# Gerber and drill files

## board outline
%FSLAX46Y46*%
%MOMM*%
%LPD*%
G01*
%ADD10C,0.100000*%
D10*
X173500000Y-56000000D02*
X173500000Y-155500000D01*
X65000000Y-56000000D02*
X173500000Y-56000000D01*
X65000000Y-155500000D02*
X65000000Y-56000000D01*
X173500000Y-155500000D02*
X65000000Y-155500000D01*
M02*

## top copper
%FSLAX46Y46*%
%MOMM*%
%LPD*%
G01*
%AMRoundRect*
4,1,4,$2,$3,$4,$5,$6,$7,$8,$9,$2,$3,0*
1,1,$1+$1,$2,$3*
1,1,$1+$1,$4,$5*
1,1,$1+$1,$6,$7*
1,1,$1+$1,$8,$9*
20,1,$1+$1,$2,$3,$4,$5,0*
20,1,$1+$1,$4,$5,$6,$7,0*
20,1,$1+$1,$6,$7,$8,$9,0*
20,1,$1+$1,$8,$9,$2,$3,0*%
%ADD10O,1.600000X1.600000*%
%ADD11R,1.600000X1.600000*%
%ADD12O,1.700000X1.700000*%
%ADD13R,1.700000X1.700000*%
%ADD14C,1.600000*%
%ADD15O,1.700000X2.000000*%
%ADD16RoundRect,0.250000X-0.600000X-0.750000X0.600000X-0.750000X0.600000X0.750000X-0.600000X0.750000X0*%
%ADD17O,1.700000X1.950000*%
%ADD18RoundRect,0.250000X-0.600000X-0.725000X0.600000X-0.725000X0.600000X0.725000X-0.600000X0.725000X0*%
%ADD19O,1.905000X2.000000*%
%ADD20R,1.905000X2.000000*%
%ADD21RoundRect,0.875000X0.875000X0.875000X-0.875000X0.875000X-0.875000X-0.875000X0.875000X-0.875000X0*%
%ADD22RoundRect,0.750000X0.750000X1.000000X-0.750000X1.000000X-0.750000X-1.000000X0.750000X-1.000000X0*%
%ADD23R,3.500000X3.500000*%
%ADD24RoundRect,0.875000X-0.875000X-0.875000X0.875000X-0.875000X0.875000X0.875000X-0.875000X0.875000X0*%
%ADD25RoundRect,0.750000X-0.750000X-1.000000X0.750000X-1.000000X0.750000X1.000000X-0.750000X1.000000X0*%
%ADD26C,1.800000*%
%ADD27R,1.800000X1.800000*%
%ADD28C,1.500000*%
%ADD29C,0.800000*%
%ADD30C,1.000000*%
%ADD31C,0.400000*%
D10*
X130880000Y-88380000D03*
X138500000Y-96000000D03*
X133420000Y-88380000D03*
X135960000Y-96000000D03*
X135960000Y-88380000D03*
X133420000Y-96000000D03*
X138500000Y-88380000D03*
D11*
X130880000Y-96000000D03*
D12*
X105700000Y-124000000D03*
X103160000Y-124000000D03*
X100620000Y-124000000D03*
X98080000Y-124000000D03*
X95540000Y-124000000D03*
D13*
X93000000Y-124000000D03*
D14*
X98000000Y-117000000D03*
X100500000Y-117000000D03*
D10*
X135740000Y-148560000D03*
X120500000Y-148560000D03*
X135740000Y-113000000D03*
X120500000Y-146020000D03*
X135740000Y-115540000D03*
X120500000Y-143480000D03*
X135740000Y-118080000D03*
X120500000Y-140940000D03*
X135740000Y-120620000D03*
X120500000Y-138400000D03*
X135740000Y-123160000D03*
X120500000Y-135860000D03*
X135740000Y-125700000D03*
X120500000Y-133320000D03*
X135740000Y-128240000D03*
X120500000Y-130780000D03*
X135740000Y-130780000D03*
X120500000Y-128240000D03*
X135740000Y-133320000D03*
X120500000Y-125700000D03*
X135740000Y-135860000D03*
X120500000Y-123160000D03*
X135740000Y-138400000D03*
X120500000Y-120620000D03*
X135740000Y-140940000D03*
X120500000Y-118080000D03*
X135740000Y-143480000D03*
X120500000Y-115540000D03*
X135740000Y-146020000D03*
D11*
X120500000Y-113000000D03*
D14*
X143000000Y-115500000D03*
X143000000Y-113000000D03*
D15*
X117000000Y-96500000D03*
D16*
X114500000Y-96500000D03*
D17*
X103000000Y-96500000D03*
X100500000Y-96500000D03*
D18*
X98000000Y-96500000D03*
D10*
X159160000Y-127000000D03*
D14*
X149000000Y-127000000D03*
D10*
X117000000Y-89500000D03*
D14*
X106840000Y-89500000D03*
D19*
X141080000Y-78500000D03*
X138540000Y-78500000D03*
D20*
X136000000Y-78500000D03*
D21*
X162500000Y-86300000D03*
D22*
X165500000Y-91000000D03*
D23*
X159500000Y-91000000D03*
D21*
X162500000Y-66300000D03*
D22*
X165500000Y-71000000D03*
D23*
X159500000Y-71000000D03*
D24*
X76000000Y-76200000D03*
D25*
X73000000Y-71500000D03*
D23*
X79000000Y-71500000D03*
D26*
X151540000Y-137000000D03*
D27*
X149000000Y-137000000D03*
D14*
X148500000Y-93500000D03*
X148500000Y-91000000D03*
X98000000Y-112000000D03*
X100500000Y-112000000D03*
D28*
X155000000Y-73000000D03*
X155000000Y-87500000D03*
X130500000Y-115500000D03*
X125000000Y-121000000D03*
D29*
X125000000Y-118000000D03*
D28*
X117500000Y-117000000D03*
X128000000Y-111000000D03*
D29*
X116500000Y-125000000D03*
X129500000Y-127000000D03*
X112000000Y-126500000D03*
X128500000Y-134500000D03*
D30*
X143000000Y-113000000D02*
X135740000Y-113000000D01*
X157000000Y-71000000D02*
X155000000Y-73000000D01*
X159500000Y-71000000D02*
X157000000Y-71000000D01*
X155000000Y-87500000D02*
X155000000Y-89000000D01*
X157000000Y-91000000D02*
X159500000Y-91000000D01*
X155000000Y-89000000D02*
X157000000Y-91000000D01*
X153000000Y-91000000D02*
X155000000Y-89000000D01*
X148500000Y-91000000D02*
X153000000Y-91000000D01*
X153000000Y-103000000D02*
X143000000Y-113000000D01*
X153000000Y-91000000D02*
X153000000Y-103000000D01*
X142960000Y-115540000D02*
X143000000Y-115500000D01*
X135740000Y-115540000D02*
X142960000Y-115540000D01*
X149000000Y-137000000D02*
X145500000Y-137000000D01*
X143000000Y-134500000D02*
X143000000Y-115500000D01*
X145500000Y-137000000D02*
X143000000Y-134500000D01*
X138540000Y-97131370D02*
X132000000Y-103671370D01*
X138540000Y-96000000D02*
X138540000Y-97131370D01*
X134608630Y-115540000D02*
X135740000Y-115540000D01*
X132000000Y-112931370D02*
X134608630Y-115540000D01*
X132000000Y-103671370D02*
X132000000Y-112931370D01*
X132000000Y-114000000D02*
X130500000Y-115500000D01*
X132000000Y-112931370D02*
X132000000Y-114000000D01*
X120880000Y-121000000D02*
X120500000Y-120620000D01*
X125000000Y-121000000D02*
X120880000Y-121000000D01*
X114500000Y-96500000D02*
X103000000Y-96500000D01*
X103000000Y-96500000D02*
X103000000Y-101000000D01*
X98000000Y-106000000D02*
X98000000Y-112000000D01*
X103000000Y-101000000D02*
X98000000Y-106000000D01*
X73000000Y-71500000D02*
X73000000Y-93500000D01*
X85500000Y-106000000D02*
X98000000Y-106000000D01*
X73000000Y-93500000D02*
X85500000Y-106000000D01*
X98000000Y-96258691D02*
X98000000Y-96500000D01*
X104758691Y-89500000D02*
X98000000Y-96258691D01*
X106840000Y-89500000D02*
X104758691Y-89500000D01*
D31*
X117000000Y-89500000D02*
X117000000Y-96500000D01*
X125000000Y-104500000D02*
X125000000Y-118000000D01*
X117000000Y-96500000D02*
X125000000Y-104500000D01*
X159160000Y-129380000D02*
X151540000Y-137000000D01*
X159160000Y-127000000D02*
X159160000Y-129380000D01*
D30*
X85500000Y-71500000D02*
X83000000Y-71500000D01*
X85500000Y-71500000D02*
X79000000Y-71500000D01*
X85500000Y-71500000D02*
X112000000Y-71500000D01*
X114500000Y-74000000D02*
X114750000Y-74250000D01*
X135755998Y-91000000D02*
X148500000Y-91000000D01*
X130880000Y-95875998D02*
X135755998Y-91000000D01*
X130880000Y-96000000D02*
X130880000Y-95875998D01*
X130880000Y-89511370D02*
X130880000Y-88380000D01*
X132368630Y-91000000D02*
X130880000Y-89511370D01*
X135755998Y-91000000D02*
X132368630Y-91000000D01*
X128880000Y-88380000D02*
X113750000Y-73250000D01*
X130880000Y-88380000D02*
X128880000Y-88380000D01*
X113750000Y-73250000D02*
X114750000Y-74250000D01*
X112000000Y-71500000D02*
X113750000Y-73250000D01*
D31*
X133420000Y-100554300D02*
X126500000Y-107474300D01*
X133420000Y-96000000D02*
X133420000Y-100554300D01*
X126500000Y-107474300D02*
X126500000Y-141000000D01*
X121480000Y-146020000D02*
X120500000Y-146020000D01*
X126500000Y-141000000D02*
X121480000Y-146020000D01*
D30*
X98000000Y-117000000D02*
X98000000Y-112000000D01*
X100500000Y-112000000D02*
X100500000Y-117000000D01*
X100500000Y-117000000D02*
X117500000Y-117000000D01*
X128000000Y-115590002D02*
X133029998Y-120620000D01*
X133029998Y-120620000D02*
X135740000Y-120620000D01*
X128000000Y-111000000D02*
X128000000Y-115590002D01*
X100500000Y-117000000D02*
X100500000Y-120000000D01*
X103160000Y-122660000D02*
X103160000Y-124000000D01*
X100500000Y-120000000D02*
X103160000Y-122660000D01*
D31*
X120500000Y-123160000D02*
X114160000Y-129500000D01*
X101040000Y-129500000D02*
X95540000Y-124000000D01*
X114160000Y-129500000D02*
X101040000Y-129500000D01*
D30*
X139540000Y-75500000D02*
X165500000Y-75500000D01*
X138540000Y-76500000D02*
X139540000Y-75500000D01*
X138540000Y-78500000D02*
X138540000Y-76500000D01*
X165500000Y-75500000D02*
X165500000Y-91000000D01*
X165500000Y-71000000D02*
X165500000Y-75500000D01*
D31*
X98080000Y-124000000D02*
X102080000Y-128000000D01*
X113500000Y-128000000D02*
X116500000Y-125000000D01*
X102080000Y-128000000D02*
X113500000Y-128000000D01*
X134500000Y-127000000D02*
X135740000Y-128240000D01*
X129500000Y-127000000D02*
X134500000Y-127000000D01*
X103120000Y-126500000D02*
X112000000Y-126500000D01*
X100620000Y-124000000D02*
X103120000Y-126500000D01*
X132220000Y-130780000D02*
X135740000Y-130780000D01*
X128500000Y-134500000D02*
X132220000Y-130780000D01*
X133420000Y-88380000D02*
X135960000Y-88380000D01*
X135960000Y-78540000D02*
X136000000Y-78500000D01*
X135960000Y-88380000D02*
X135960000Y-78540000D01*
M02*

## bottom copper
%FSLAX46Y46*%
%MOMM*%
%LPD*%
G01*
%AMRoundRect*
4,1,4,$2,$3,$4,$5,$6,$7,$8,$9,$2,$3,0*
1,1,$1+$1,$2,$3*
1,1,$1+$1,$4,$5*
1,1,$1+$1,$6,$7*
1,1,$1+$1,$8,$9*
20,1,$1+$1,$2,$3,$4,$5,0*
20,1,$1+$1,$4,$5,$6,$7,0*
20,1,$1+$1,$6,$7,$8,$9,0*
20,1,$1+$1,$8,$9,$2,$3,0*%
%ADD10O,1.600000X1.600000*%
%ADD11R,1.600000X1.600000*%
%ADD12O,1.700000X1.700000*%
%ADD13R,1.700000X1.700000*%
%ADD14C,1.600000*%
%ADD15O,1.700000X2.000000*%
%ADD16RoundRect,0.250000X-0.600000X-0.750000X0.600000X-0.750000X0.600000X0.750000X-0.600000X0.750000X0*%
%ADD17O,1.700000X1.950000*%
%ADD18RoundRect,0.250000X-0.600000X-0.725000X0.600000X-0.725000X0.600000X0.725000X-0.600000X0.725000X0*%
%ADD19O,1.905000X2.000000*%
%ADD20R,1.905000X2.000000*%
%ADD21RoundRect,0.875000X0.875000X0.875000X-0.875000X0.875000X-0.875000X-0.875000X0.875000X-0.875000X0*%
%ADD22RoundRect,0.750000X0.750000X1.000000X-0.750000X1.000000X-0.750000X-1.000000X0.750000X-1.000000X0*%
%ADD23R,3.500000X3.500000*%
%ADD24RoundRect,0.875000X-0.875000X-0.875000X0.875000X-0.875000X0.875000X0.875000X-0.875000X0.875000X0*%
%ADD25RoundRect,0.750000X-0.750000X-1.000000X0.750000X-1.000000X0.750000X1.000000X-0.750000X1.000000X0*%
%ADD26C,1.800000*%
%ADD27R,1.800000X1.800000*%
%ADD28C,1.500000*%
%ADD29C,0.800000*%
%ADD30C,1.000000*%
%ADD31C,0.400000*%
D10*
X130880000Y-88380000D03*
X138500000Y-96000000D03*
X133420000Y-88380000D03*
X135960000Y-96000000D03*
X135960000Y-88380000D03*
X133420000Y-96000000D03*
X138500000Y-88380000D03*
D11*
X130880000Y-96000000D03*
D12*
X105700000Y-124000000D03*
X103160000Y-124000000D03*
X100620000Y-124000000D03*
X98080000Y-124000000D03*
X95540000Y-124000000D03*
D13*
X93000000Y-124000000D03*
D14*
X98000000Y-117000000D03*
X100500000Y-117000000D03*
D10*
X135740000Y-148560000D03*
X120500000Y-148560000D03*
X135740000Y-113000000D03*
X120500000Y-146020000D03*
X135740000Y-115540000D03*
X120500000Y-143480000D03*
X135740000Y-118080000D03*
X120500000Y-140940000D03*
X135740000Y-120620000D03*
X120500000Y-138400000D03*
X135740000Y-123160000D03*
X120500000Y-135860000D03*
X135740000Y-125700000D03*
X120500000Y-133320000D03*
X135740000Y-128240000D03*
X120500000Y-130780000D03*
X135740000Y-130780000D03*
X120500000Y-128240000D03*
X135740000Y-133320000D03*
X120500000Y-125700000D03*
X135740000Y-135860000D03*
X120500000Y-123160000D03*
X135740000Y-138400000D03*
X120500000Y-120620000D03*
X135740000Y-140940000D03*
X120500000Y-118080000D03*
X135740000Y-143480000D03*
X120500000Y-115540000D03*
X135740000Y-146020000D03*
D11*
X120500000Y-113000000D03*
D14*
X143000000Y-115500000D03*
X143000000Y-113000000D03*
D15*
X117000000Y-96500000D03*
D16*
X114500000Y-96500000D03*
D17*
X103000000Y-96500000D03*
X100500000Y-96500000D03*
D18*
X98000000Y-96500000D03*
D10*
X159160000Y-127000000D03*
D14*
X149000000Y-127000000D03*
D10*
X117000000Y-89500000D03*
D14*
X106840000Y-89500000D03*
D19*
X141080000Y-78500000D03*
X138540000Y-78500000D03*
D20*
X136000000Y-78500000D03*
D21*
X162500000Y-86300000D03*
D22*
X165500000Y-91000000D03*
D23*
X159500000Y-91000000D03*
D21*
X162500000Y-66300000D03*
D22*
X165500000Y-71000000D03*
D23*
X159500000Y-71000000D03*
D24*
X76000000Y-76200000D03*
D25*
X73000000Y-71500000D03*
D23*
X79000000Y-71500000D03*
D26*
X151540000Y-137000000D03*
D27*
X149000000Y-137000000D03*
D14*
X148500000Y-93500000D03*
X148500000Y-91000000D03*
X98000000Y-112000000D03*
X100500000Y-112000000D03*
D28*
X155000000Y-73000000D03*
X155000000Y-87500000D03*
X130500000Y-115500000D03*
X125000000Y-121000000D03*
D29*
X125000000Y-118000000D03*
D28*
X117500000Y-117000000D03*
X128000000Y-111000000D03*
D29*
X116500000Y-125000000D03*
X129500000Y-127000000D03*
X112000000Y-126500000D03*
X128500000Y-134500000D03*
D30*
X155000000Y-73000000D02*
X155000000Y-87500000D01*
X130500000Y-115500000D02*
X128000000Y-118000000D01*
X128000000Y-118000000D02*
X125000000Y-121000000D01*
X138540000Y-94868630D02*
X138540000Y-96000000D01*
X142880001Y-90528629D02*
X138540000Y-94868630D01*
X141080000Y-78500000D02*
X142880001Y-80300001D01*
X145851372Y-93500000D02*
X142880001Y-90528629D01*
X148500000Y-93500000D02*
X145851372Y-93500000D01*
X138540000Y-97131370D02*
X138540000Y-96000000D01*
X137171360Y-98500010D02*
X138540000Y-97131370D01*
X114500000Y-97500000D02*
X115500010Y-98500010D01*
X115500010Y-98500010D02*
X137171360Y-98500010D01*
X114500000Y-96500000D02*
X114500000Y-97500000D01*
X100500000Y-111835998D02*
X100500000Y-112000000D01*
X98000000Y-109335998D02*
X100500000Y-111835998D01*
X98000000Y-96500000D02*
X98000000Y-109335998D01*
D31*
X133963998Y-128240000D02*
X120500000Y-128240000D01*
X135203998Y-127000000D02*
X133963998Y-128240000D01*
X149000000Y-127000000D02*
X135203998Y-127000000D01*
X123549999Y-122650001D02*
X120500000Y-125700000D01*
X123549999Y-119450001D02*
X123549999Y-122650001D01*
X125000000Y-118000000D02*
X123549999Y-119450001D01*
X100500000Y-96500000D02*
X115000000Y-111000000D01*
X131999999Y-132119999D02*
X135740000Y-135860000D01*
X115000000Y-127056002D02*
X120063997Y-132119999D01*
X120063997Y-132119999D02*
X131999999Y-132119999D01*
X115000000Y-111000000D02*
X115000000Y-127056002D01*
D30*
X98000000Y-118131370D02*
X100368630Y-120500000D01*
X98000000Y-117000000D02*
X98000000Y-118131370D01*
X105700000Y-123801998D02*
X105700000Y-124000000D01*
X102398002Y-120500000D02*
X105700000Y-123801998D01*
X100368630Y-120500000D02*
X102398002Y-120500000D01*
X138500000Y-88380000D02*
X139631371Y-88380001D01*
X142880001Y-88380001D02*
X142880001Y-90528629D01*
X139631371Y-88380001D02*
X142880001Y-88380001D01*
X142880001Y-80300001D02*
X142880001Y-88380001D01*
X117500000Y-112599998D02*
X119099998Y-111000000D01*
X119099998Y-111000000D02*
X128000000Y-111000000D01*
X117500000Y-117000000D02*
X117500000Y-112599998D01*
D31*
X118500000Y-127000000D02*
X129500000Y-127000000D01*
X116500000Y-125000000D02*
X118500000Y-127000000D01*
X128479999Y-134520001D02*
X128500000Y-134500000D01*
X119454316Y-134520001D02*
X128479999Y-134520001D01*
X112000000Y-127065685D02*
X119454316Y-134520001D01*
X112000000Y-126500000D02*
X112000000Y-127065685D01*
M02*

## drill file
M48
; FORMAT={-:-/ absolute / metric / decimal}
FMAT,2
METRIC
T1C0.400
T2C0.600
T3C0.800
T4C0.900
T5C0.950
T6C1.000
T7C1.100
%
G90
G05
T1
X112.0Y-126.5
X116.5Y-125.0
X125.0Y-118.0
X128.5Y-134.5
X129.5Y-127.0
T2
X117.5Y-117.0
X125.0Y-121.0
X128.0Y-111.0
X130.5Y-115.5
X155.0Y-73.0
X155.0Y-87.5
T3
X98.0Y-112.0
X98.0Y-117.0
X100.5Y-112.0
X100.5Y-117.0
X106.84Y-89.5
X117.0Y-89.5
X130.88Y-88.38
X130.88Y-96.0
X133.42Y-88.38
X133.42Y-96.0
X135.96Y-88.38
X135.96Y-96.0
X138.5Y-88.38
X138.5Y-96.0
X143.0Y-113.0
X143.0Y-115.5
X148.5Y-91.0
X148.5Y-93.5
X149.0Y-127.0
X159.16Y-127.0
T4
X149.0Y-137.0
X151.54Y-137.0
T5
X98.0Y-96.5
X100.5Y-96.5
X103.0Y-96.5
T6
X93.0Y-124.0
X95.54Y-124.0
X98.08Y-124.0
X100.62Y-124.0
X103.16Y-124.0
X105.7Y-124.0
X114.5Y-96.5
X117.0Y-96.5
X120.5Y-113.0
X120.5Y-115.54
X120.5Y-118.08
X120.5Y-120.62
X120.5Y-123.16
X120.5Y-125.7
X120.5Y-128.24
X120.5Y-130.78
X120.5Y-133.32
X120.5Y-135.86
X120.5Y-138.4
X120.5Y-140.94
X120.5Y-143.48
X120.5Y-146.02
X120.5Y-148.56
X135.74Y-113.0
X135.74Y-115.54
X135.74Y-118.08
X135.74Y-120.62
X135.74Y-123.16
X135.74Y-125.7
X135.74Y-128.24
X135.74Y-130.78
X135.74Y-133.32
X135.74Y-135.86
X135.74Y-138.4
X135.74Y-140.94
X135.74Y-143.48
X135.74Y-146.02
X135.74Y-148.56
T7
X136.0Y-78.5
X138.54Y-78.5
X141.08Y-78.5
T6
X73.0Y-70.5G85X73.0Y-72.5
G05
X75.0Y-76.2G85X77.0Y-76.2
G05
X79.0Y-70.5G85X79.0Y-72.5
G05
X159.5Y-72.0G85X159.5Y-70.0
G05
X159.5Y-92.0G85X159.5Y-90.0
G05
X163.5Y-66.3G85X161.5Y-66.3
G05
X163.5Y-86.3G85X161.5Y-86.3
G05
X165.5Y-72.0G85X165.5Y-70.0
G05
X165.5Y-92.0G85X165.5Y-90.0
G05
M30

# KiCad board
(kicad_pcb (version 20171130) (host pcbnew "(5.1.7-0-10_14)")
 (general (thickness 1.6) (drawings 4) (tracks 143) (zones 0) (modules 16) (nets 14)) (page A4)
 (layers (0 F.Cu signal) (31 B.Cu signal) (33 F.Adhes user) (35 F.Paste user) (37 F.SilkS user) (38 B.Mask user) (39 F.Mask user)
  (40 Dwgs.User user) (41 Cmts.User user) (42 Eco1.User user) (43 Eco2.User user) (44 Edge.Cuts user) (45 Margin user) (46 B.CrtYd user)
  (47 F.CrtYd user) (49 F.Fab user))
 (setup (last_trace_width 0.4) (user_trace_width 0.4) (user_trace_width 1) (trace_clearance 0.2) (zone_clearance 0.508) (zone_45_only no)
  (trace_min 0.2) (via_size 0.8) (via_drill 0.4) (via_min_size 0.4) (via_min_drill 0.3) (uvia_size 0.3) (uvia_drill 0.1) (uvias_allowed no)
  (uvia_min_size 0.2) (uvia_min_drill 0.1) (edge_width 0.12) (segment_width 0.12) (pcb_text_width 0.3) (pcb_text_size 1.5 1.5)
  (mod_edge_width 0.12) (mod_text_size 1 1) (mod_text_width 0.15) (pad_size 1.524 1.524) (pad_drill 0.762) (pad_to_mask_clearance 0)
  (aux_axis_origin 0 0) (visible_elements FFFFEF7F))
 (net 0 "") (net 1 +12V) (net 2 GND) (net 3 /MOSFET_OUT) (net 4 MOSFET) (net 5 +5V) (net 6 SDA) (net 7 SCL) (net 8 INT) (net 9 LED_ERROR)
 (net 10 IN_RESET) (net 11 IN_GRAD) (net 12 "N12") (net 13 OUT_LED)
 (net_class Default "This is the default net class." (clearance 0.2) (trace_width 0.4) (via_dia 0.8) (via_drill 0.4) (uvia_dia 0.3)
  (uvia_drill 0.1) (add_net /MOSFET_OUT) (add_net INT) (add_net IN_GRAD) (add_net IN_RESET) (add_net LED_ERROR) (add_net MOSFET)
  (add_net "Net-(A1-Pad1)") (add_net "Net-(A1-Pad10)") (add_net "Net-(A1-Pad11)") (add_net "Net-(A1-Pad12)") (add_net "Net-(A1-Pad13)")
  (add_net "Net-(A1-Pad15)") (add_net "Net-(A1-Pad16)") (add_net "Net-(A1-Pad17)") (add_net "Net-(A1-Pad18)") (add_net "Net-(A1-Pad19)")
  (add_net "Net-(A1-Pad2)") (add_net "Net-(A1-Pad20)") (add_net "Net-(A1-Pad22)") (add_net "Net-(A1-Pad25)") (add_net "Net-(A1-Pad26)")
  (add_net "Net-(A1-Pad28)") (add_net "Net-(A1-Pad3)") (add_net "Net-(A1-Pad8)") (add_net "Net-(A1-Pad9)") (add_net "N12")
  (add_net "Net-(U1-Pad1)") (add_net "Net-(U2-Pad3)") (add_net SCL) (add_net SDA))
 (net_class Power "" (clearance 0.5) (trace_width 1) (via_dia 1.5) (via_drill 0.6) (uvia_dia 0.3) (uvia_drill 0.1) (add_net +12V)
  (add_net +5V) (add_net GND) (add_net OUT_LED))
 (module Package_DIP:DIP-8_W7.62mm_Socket (layer F.Cu) (at 130.88 96 90)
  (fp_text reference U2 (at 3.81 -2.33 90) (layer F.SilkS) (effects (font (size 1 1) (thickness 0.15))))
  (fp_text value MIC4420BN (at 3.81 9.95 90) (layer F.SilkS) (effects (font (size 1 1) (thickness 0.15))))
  (pad 8 thru_hole oval (at 7.62 0 90) (size 1.6 1.6) (drill 0.8) (layers *.Cu *.Mask) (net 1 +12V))
  (pad 4 thru_hole oval (at 0 7.62 90) (size 1.6 1.6) (drill 0.8) (layers *.Cu *.Mask) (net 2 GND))
  (pad 7 thru_hole oval (at 7.62 2.54 90) (size 1.6 1.6) (drill 0.8) (layers *.Cu *.Mask) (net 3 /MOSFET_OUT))
  (pad 3 thru_hole oval (at 0 5.08 90) (size 1.6 1.6) (drill 0.8) (layers *.Cu *.Mask))
  (pad 6 thru_hole oval (at 7.62 5.08 90) (size 1.6 1.6) (drill 0.8) (layers *.Cu *.Mask) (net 3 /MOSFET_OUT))
  (pad 2 thru_hole oval (at 0 2.54 90) (size 1.6 1.6) (drill 0.8) (layers *.Cu *.Mask) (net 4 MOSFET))
  (pad 5 thru_hole oval (at 7.62 7.62 90) (size 1.6 1.6) (drill 0.8) (layers *.Cu *.Mask) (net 2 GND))
  (pad 1 thru_hole rect (at 0 0 90) (size 1.6 1.6) (drill 0.8) (layers *.Cu *.Mask) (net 1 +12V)))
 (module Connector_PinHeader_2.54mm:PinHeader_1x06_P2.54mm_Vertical (layer F.Cu) (at 93 124 90)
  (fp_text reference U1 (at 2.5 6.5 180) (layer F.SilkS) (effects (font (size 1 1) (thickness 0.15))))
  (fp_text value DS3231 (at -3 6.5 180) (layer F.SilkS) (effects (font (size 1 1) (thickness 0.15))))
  (pad 6 thru_hole oval (at 0 12.7 90) (size 1.7 1.7) (drill 1) (layers *.Cu *.Mask) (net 2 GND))
  (pad 5 thru_hole oval (at 0 10.16 90) (size 1.7 1.7) (drill 1) (layers *.Cu *.Mask) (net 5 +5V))
  (pad 4 thru_hole oval (at 0 7.62 90) (size 1.7 1.7) (drill 1) (layers *.Cu *.Mask) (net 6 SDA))
  (pad 3 thru_hole oval (at 0 5.08 90) (size 1.7 1.7) (drill 1) (layers *.Cu *.Mask) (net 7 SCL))
  (pad 2 thru_hole oval (at 0 2.54 90) (size 1.7 1.7) (drill 1) (layers *.Cu *.Mask) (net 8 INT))
  (pad 1 thru_hole rect (at 0 0 90) (size 1.7 1.7) (drill 1) (layers *.Cu *.Mask)))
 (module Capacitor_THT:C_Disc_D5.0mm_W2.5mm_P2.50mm (layer F.Cu) (at 100.5 117 180)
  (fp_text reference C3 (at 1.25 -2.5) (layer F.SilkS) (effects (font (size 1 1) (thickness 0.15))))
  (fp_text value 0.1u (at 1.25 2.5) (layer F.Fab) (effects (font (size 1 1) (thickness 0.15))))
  (pad 2 thru_hole circle (at 2.5 0 180) (size 1.6 1.6) (drill 0.8) (layers *.Cu *.Mask) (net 2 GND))
  (pad 1 thru_hole circle (at 0 0 180) (size 1.6 1.6) (drill 0.8) (layers *.Cu *.Mask) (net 5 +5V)))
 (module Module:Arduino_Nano (layer F.Cu) (at 120.5 113)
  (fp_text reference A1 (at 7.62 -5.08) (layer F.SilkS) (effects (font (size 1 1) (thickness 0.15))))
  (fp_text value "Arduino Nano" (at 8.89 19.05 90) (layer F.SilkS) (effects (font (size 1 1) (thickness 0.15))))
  (pad 16 thru_hole oval (at 15.24 35.56) (size 1.6 1.6) (drill 1) (layers *.Cu *.Mask))
  (pad 15 thru_hole oval (at 0 35.56) (size 1.6 1.6) (drill 1) (layers *.Cu *.Mask))
  (pad 30 thru_hole oval (at 15.24 0) (size 1.6 1.6) (drill 1) (layers *.Cu *.Mask) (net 1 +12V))
  (pad 14 thru_hole oval (at 0 33.02) (size 1.6 1.6) (drill 1) (layers *.Cu *.Mask) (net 4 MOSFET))
  (pad 29 thru_hole oval (at 15.24 2.54) (size 1.6 1.6) (drill 1) (layers *.Cu *.Mask) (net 2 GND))
  (pad 13 thru_hole oval (at 0 30.48) (size 1.6 1.6) (drill 1) (layers *.Cu *.Mask))
  (pad 28 thru_hole oval (at 15.24 5.08) (size 1.6 1.6) (drill 1) (layers *.Cu *.Mask))
  (pad 12 thru_hole oval (at 0 27.94) (size 1.6 1.6) (drill 1) (layers *.Cu *.Mask))
  (pad 27 thru_hole oval (at 15.24 7.62) (size 1.6 1.6) (drill 1) (layers *.Cu *.Mask) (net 5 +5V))
  (pad 11 thru_hole oval (at 0 25.4) (size 1.6 1.6) (drill 1) (layers *.Cu *.Mask))
  (pad 26 thru_hole oval (at 15.24 10.16) (size 1.6 1.6) (drill 1) (layers *.Cu *.Mask))
  (pad 10 thru_hole oval (at 0 22.86) (size 1.6 1.6) (drill 1) (layers *.Cu *.Mask))
  (pad 25 thru_hole oval (at 15.24 12.7) (size 1.6 1.6) (drill 1) (layers *.Cu *.Mask))
  (pad 9 thru_hole oval (at 0 20.32) (size 1.6 1.6) (drill 1) (layers *.Cu *.Mask))
  (pad 24 thru_hole oval (at 15.24 15.24) (size 1.6 1.6) (drill 1) (layers *.Cu *.Mask) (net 7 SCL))
  (pad 8 thru_hole oval (at 0 17.78) (size 1.6 1.6) (drill 1) (layers *.Cu *.Mask))
  (pad 23 thru_hole oval (at 15.24 17.78) (size 1.6 1.6) (drill 1) (layers *.Cu *.Mask) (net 6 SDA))
  (pad 7 thru_hole oval (at 0 15.24) (size 1.6 1.6) (drill 1) (layers *.Cu *.Mask) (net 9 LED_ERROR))
  (pad 22 thru_hole oval (at 15.24 20.32) (size 1.6 1.6) (drill 1) (layers *.Cu *.Mask))
  (pad 6 thru_hole oval (at 0 12.7) (size 1.6 1.6) (drill 1) (layers *.Cu *.Mask) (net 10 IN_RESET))
  (pad 21 thru_hole oval (at 15.24 22.86) (size 1.6 1.6) (drill 1) (layers *.Cu *.Mask) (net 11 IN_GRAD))
  (pad 5 thru_hole oval (at 0 10.16) (size 1.6 1.6) (drill 1) (layers *.Cu *.Mask) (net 8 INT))
  (pad 20 thru_hole oval (at 15.24 25.4) (size 1.6 1.6) (drill 1) (layers *.Cu *.Mask))
  (pad 4 thru_hole oval (at 0 7.62) (size 1.6 1.6) (drill 1) (layers *.Cu *.Mask) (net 2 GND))
  (pad 19 thru_hole oval (at 15.24 27.94) (size 1.6 1.6) (drill 1) (layers *.Cu *.Mask))
  (pad 3 thru_hole oval (at 0 5.08) (size 1.6 1.6) (drill 1) (layers *.Cu *.Mask))
  (pad 18 thru_hole oval (at 15.24 30.48) (size 1.6 1.6) (drill 1) (layers *.Cu *.Mask))
  (pad 2 thru_hole oval (at 0 2.54) (size 1.6 1.6) (drill 1) (layers *.Cu *.Mask))
  (pad 17 thru_hole oval (at 15.24 33.02) (size 1.6 1.6) (drill 1) (layers *.Cu *.Mask))
  (pad 1 thru_hole rect (at 0 0) (size 1.6 1.6) (drill 1) (layers *.Cu *.Mask)))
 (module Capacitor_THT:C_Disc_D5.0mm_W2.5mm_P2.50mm (layer F.Cu) (at 143 113 270)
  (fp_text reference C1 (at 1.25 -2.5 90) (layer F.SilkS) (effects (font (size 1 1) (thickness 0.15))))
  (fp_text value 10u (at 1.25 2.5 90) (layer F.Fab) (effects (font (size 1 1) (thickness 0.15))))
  (pad 2 thru_hole circle (at 2.5 0 270) (size 1.6 1.6) (drill 0.8) (layers *.Cu *.Mask) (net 2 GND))
  (pad 1 thru_hole circle (at 0 0 270) (size 1.6 1.6) (drill 0.8) (layers *.Cu *.Mask) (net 1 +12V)))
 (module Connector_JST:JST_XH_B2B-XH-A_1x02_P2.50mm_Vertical (layer F.Cu) (at 114.5 96.5)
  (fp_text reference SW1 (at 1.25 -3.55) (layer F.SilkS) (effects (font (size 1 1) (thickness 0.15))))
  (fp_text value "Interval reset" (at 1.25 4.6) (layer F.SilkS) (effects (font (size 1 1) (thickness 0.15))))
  (pad 2 thru_hole oval (at 2.5 0) (size 1.7 2) (drill 1) (layers *.Cu *.Mask) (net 10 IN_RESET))
  (pad 1 thru_hole roundrect (at 0 0) (size 1.7 2) (drill 1) (layers *.Cu *.Mask) (roundrect_rratio 0.147059) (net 2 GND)))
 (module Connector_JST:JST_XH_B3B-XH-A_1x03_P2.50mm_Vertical (layer F.Cu) (at 98 96.5)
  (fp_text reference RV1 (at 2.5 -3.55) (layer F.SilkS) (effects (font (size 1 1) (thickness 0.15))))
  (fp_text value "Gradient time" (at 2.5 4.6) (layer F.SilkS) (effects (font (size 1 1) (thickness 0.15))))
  (pad 3 thru_hole oval (at 5 0) (size 1.7 1.95) (drill 0.95) (layers *.Cu *.Mask) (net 2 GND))
  (pad 2 thru_hole oval (at 2.5 0) (size 1.7 1.95) (drill 0.95) (layers *.Cu *.Mask) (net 11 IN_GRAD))
  (pad 1 thru_hole roundrect (at 0 0) (size 1.7 1.95) (drill 0.95) (layers *.Cu *.Mask) (roundrect_rratio 0.147059) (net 5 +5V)))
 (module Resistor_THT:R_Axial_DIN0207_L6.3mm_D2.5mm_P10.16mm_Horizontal (layer F.Cu) (at 149 127)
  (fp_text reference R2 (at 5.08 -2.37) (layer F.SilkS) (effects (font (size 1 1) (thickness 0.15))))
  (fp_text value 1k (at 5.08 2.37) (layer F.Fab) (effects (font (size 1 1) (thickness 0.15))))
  (pad 2 thru_hole oval (at 10.16 0) (size 1.6 1.6) (drill 0.8) (layers *.Cu *.Mask) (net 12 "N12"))
  (pad 1 thru_hole circle (at 0 0) (size 1.6 1.6) (drill 0.8) (layers *.Cu *.Mask) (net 9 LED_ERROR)))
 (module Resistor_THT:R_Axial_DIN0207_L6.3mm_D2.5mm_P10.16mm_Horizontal (layer F.Cu) (at 106.84 89.5)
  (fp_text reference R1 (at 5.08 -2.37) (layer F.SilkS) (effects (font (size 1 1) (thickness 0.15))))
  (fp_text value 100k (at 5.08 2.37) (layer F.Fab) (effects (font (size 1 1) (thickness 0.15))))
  (pad 2 thru_hole oval (at 10.16 0) (size 1.6 1.6) (drill 0.8) (layers *.Cu *.Mask) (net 10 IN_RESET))
  (pad 1 thru_hole circle (at 0 0) (size 1.6 1.6) (drill 0.8) (layers *.Cu *.Mask) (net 5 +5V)))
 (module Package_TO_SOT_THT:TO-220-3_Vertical (layer F.Cu) (at 136 78.5)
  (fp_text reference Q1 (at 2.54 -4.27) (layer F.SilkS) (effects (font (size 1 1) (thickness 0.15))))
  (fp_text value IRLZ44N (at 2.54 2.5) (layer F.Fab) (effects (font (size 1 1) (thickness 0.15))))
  (pad 3 thru_hole oval (at 5.08 0) (size 1.905 2) (drill 1.1) (layers *.Cu *.Mask) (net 2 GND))
  (pad 2 thru_hole oval (at 2.54 0) (size 1.905 2) (drill 1.1) (layers *.Cu *.Mask) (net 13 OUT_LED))
  (pad 1 thru_hole rect (at 0 0) (size 1.905 2) (drill 1.1) (layers *.Cu *.Mask) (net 3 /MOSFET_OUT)))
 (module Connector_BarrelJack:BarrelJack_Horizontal (layer F.Cu) (at 159.5 91 180)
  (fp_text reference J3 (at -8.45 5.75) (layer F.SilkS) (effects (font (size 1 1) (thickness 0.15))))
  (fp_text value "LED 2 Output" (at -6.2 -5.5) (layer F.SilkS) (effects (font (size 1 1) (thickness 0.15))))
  (pad 3 thru_hole roundrect (at -3 4.7 180) (size 3.5 3.5) (drill oval 3 1) (layers *.Cu *.Mask) (roundrect_rratio 0.25))
  (pad 2 thru_hole roundrect (at -6 0 180) (size 3 3.5) (drill oval 1 3) (layers *.Cu *.Mask) (roundrect_rratio 0.25) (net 13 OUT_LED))
  (pad 1 thru_hole rect (at 0 0 180) (size 3.5 3.5) (drill oval 1 3) (layers *.Cu *.Mask) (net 1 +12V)))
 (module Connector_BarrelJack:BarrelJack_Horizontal (layer F.Cu) (at 159.5 71 180)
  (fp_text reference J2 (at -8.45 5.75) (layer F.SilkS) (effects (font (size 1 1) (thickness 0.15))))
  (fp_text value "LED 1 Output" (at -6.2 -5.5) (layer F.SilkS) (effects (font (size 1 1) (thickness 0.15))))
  (pad 3 thru_hole roundrect (at -3 4.7 180) (size 3.5 3.5) (drill oval 3 1) (layers *.Cu *.Mask) (roundrect_rratio 0.25))
  (pad 2 thru_hole roundrect (at -6 0 180) (size 3 3.5) (drill oval 1 3) (layers *.Cu *.Mask) (roundrect_rratio 0.25) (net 13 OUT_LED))
  (pad 1 thru_hole rect (at 0 0 180) (size 3.5 3.5) (drill oval 1 3) (layers *.Cu *.Mask) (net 1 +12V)))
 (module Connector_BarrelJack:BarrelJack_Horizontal (layer F.Cu) (at 79 71.5)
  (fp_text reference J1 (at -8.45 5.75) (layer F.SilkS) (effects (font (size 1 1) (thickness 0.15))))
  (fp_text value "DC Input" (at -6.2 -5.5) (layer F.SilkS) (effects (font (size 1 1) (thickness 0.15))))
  (pad 3 thru_hole roundrect (at -3 4.7) (size 3.5 3.5) (drill oval 3 1) (layers *.Cu *.Mask) (roundrect_rratio 0.25))
  (pad 2 thru_hole roundrect (at -6 0) (size 3 3.5) (drill oval 1 3) (layers *.Cu *.Mask) (roundrect_rratio 0.25) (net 2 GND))
  (pad 1 thru_hole rect (at 0 0) (size 3.5 3.5) (drill oval 1 3) (layers *.Cu *.Mask) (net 1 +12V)))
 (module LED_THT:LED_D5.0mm (layer F.Cu) (at 149 137)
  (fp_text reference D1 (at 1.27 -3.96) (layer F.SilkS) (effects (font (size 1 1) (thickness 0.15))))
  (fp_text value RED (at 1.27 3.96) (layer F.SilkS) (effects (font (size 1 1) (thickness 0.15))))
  (pad 2 thru_hole circle (at 2.54 0) (size 1.8 1.8) (drill 0.9) (layers *.Cu *.Mask) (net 12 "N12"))
  (pad 1 thru_hole rect (at 0 0) (size 1.8 1.8) (drill 0.9) (layers *.Cu *.Mask) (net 2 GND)))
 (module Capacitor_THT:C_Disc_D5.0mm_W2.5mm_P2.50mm (layer F.Cu) (at 148.5 91 270)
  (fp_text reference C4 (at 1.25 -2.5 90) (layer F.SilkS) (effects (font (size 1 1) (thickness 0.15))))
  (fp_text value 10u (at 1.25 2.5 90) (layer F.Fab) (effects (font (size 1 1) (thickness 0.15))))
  (pad 2 thru_hole circle (at 2.5 0 270) (size 1.6 1.6) (drill 0.8) (layers *.Cu *.Mask) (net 2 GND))
  (pad 1 thru_hole circle (at 0 0 270) (size 1.6 1.6) (drill 0.8) (layers *.Cu *.Mask) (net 1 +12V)))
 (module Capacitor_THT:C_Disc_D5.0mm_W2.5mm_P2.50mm (layer F.Cu) (at 100.5 112 180)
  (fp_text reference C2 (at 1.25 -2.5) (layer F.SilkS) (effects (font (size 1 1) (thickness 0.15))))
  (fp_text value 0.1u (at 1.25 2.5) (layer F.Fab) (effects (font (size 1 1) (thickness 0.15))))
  (pad 2 thru_hole circle (at 2.5 0 180) (size 1.6 1.6) (drill 0.8) (layers *.Cu *.Mask) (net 2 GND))
  (pad 1 thru_hole circle (at 0 0 180) (size 1.6 1.6) (drill 0.8) (layers *.Cu *.Mask) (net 5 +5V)))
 (gr_line (start 173.5 56) (end 173.5 155.5) (layer Edge.Cuts) (width 0.1))
 (gr_line (start 65 56) (end 173.5 56) (layer Edge.Cuts) (width 0.1))
 (gr_line (start 65 155.5) (end 65 56) (layer Edge.Cuts) (width 0.1))
 (gr_line (start 173.5 155.5) (end 65 155.5) (layer Edge.Cuts) (width 0.1))
 (segment (start 143 113) (end 135.74 113) (width 1) (layer F.Cu) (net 1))
 (via (at 155 73) (size 1.5) (drill 0.6) (layers F.Cu B.Cu) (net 1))
 (segment (start 157 71) (end 155 73) (width 1) (layer F.Cu) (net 1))
 (segment (start 159.5 71) (end 157 71) (width 1) (layer F.Cu) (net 1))
 (via (at 155 87.5) (size 1.5) (drill 0.6) (layers F.Cu B.Cu) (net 1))
 (segment (start 155 73) (end 155 87.5) (width 1) (layer B.Cu) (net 1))
 (segment (start 155 87.5) (end 155 89) (width 1) (layer F.Cu) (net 1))
 (segment (start 157 91) (end 159.5 91) (width 1) (layer F.Cu) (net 1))
 (segment (start 155 89) (end 157 91) (width 1) (layer F.Cu) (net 1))
 (segment (start 153 91) (end 155 89) (width 1) (layer F.Cu) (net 1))
 (segment (start 148.5 91) (end 153 91) (width 1) (layer F.Cu) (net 1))
 (segment (start 153 103) (end 143 113) (width 1) (layer F.Cu) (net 1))
 (segment (start 153 91) (end 153 103) (width 1) (layer F.Cu) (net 1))
 (segment (start 142.96 115.54) (end 143 115.5) (width 1) (layer F.Cu) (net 2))
 (segment (start 135.74 115.54) (end 142.96 115.54) (width 1) (layer F.Cu) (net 2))
 (segment (start 149 137) (end 145.5 137) (width 1) (layer F.Cu) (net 2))
 (segment (start 143 134.5) (end 143 115.5) (width 1) (layer F.Cu) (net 2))
 (segment (start 145.5 137) (end 143 134.5) (width 1) (layer F.Cu) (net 2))
 (segment (start 138.54 97.13137) (end 132 103.67137) (width 1) (layer F.Cu) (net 2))
 (segment (start 138.54 96) (end 138.54 97.13137) (width 1) (layer F.Cu) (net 2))
 (segment (start 134.60863 115.54) (end 135.74 115.54) (width 1) (layer F.Cu) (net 2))
 (segment (start 132 112.93137) (end 134.60863 115.54) (width 1) (layer F.Cu) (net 2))
 (segment (start 132 103.67137) (end 132 112.93137) (width 1) (layer F.Cu) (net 2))
 (via (at 130.5 115.5) (size 1.5) (drill 0.6) (layers F.Cu B.Cu) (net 2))
 (segment (start 132 114) (end 130.5 115.5) (width 1) (layer F.Cu) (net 2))
 (segment (start 132 112.93137) (end 132 114) (width 1) (layer F.Cu) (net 2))
 (segment (start 130.5 115.5) (end 128 118) (width 1) (layer B.Cu) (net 2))
 (via (at 125 121) (size 1.5) (drill 0.6) (layers F.Cu B.Cu) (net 2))
 (segment (start 128 118) (end 125 121) (width 1) (layer B.Cu) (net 2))
 (segment (start 120.88 121) (end 120.5 120.62) (width 1) (layer F.Cu) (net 2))
 (segment (start 125 121) (end 120.88 121) (width 1) (layer F.Cu) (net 2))
 (segment (start 114.5 96.5) (end 103 96.5) (width 1) (layer F.Cu) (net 2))
 (segment (start 103 96.5) (end 103 101) (width 1) (layer F.Cu) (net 2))
 (segment (start 98 106) (end 98 112) (width 1) (layer F.Cu) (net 2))
 (segment (start 103 101) (end 98 106) (width 1) (layer F.Cu) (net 2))
 (segment (start 73 71.5) (end 73 93.5) (width 1) (layer F.Cu) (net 2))
 (segment (start 85.5 106) (end 98 106) (width 1) (layer F.Cu) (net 2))
 (segment (start 73 93.5) (end 85.5 106) (width 1) (layer F.Cu) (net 2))
 (segment (start 138.54 94.86863) (end 138.54 96) (width 1) (layer B.Cu) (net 2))
 (segment (start 142.880001 90.528629) (end 138.54 94.86863) (width 1) (layer B.Cu) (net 2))
 (segment (start 141.08 78.5) (end 142.880001 80.300001) (width 1) (layer B.Cu) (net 2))
 (segment (start 145.851372 93.5) (end 142.880001 90.528629) (width 1) (layer B.Cu) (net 2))
 (segment (start 148.5 93.5) (end 145.851372 93.5) (width 1) (layer B.Cu) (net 2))
 (segment (start 138.54 97.13137) (end 138.54 96) (width 1) (layer B.Cu) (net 2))
 (segment (start 137.17136 98.50001) (end 138.54 97.13137) (width 1) (layer B.Cu) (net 2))
 (segment (start 114.5 97.5) (end 115.50001 98.50001) (width 1) (layer B.Cu) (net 2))
 (segment (start 115.50001 98.50001) (end 137.17136 98.50001) (width 1) (layer B.Cu) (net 2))
 (segment (start 114.5 96.5) (end 114.5 97.5) (width 1) (layer B.Cu) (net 2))
 (segment (start 98 96.258691) (end 98 96.5) (width 1) (layer F.Cu) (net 5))
 (segment (start 104.758691 89.5) (end 98 96.258691) (width 1) (layer F.Cu) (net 5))
 (segment (start 106.84 89.5) (end 104.758691 89.5) (width 1) (layer F.Cu) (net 5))
 (segment (start 100.5 111.835998) (end 100.5 112) (width 1) (layer B.Cu) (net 5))
 (segment (start 98 109.335998) (end 100.5 111.835998) (width 1) (layer B.Cu) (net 5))
 (segment (start 98 96.5) (end 98 109.335998) (width 1) (layer B.Cu) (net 5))
 (segment (start 133.963998 128.24) (end 120.5 128.24) (width 0.4) (layer B.Cu) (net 9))
 (segment (start 135.203998 127) (end 133.963998 128.24) (width 0.4) (layer B.Cu) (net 9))
 (segment (start 149 127) (end 135.203998 127) (width 0.4) (layer B.Cu) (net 9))
 (segment (start 117 89.5) (end 117 96.5) (width 0.4) (layer F.Cu) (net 10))
 (via (at 125 118) (size 0.8) (drill 0.4) (layers F.Cu B.Cu) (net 10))
 (segment (start 125 104.5) (end 125 118) (width 0.4) (layer F.Cu) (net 10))
 (segment (start 117 96.5) (end 125 104.5) (width 0.4) (layer F.Cu) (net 10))
 (segment (start 123.549999 122.650001) (end 120.5 125.7) (width 0.4) (layer B.Cu) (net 10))
 (segment (start 123.549999 119.450001) (end 123.549999 122.650001) (width 0.4) (layer B.Cu) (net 10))
 (segment (start 125 118) (end 123.549999 119.450001) (width 0.4) (layer B.Cu) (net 10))
 (segment (start 100.5 96.5) (end 115 111) (width 0.4) (layer B.Cu) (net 11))
 (segment (start 131.999999 132.119999) (end 135.74 135.86) (width 0.4) (layer B.Cu) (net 11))
 (segment (start 115 127.056002) (end 120.063997 132.119999) (width 0.4) (layer B.Cu) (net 11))
 (segment (start 120.063997 132.119999) (end 131.999999 132.119999) (width 0.4) (layer B.Cu) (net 11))
 (segment (start 115 111) (end 115 127.056002) (width 0.4) (layer B.Cu) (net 11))
 (segment (start 159.16 129.38) (end 151.54 137) (width 0.4) (layer F.Cu) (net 12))
 (segment (start 159.16 127) (end 159.16 129.38) (width 0.4) (layer F.Cu) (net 12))
 (segment (start 85.5 71.5) (end 83 71.5) (width 1) (layer F.Cu) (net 1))
 (segment (start 85.5 71.5) (end 79 71.5) (width 1) (layer F.Cu) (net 1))
 (segment (start 85.5 71.5) (end 112 71.5) (width 1) (layer F.Cu) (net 1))
 (segment (start 114.5 74) (end 114.75 74.25) (width 1) (layer F.Cu) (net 1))
 (segment (start 135.755998 91) (end 148.5 91) (width 1) (layer F.Cu) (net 1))
 (segment (start 130.88 95.875998) (end 135.755998 91) (width 1) (layer F.Cu) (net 1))
 (segment (start 130.88 96) (end 130.88 95.875998) (width 1) (layer F.Cu) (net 1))
 (segment (start 130.88 89.51137) (end 130.88 88.38) (width 1) (layer F.Cu) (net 1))
 (segment (start 132.36863 91) (end 130.88 89.51137) (width 1) (layer F.Cu) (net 1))
 (segment (start 135.755998 91) (end 132.36863 91) (width 1) (layer F.Cu) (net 1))
 (segment (start 128.88 88.38) (end 113.75 73.25) (width 1) (layer F.Cu) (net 1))
 (segment (start 130.88 88.38) (end 128.88 88.38) (width 1) (layer F.Cu) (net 1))
 (segment (start 113.75 73.25) (end 114.75 74.25) (width 1) (layer F.Cu) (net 1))
 (segment (start 112 71.5) (end 113.75 73.25) (width 1) (layer F.Cu) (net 1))
 (segment (start 133.42 100.5543) (end 126.5 107.4743) (width 0.4) (layer F.Cu) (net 4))
 (segment (start 133.42 96) (end 133.42 100.5543) (width 0.4) (layer F.Cu) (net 4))
 (segment (start 126.5 107.4743) (end 126.5 141) (width 0.4) (layer F.Cu) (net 4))
 (segment (start 121.48 146.02) (end 120.5 146.02) (width 0.4) (layer F.Cu) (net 4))
 (segment (start 126.5 141) (end 121.48 146.02) (width 0.4) (layer F.Cu) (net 4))
 (segment (start 98 117) (end 98 112) (width 1) (layer F.Cu) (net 2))
 (segment (start 98 118.13137) (end 100.36863 120.5) (width 1) (layer B.Cu) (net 2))
 (segment (start 98 117) (end 98 118.13137) (width 1) (layer B.Cu) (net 2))
 (segment (start 105.7 123.801998) (end 105.7 124) (width 1) (layer B.Cu) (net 2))
 (segment (start 102.398002 120.5) (end 105.7 123.801998) (width 1) (layer B.Cu) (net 2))
 (segment (start 100.36863 120.5) (end 102.398002 120.5) (width 1) (layer B.Cu) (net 2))
 (segment (start 138.5 88.38) (end 139.631371 88.380001) (width 1) (layer B.Cu) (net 2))
 (segment (start 142.880001 88.380001) (end 142.880001 90.528629) (width 1) (layer B.Cu) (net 2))
 (segment (start 139.631371 88.380001) (end 142.880001 88.380001) (width 1) (layer B.Cu) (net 2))
 (segment (start 142.880001 80.300001) (end 142.880001 88.380001) (width 1) (layer B.Cu) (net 2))
 (segment (start 100.5 112) (end 100.5 117) (width 1) (layer F.Cu) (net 5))
 (via (at 117.5 117) (size 1.5) (drill 0.6) (layers F.Cu B.Cu) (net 5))
 (segment (start 100.5 117) (end 117.5 117) (width 1) (layer F.Cu) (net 5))
 (segment (start 117.5 112.599998) (end 119.099998 111) (width 1) (layer B.Cu) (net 5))
 (via (at 128 111) (size 1.5) (drill 0.6) (layers F.Cu B.Cu) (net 5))
 (segment (start 119.099998 111) (end 128 111) (width 1) (layer B.Cu) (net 5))
 (segment (start 117.5 117) (end 117.5 112.599998) (width 1) (layer B.Cu) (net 5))
 (segment (start 128 115.590002) (end 133.029998 120.62) (width 1) (layer F.Cu) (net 5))
 (segment (start 133.029998 120.62) (end 135.74 120.62) (width 1) (layer F.Cu) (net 5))
 (segment (start 128 111) (end 128 115.590002) (width 1) (layer F.Cu) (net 5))
 (segment (start 100.5 117) (end 100.5 120) (width 1) (layer F.Cu) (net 5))
 (segment (start 103.16 122.66) (end 103.16 124) (width 1) (layer F.Cu) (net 5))
 (segment (start 100.5 120) (end 103.16 122.66) (width 1) (layer F.Cu) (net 5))
 (segment (start 120.5 123.16) (end 114.16 129.5) (width 0.4) (layer F.Cu) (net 8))
 (segment (start 101.04 129.5) (end 95.54 124) (width 0.4) (layer F.Cu) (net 8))
 (segment (start 114.16 129.5) (end 101.04 129.5) (width 0.4) (layer F.Cu) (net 8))
 (segment (start 139.54 75.5) (end 165.5 75.5) (width 1) (layer F.Cu) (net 13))
 (segment (start 138.54 76.5) (end 139.54 75.5) (width 1) (layer F.Cu) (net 13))
 (segment (start 138.54 78.5) (end 138.54 76.5) (width 1) (layer F.Cu) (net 13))
 (segment (start 165.5 75.5) (end 165.5 91) (width 1) (layer F.Cu) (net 13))
 (segment (start 165.5 71) (end 165.5 75.5) (width 1) (layer F.Cu) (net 13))
 (segment (start 98.08 124) (end 102.08 128) (width 0.4) (layer F.Cu) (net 7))
 (via (at 116.5 125) (size 0.8) (drill 0.4) (layers F.Cu B.Cu) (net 7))
 (segment (start 113.5 128) (end 116.5 125) (width 0.4) (layer F.Cu) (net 7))
 (segment (start 102.08 128) (end 113.5 128) (width 0.4) (layer F.Cu) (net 7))
 (via (at 129.5 127) (size 0.8) (drill 0.4) (layers F.Cu B.Cu) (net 7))
 (segment (start 118.5 127) (end 129.5 127) (width 0.4) (layer B.Cu) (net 7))
 (segment (start 116.5 125) (end 118.5 127) (width 0.4) (layer B.Cu) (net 7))
 (segment (start 134.5 127) (end 135.74 128.24) (width 0.4) (layer F.Cu) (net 7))
 (segment (start 129.5 127) (end 134.5 127) (width 0.4) (layer F.Cu) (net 7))
 (via (at 112 126.5) (size 0.8) (drill 0.4) (layers F.Cu B.Cu) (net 6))
 (segment (start 103.12 126.5) (end 112 126.5) (width 0.4) (layer F.Cu) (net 6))
 (segment (start 100.62 124) (end 103.12 126.5) (width 0.4) (layer F.Cu) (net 6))
 (segment (start 128.479999 134.520001) (end 128.5 134.5) (width 0.4) (layer B.Cu) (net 6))
 (via (at 128.5 134.5) (size 0.8) (drill 0.4) (layers F.Cu B.Cu) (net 6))
 (segment (start 119.454316 134.520001) (end 128.479999 134.520001) (width 0.4) (layer B.Cu) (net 6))
 (segment (start 112 127.065685) (end 119.454316 134.520001) (width 0.4) (layer B.Cu) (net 6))
 (segment (start 112 126.5) (end 112 127.065685) (width 0.4) (layer B.Cu) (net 6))
 (segment (start 132.22 130.78) (end 135.74 130.78) (width 0.4) (layer F.Cu) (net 6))
 (segment (start 128.5 134.5) (end 132.22 130.78) (width 0.4) (layer F.Cu) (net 6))
 (segment (start 133.42 88.38) (end 135.96 88.38) (width 0.4) (layer F.Cu) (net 3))
 (segment (start 135.96 78.54) (end 136 78.5) (width 0.4) (layer F.Cu) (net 3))
 (segment (start 135.96 88.38) (end 135.96 78.54) (width 0.4) (layer F.Cu) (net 3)))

